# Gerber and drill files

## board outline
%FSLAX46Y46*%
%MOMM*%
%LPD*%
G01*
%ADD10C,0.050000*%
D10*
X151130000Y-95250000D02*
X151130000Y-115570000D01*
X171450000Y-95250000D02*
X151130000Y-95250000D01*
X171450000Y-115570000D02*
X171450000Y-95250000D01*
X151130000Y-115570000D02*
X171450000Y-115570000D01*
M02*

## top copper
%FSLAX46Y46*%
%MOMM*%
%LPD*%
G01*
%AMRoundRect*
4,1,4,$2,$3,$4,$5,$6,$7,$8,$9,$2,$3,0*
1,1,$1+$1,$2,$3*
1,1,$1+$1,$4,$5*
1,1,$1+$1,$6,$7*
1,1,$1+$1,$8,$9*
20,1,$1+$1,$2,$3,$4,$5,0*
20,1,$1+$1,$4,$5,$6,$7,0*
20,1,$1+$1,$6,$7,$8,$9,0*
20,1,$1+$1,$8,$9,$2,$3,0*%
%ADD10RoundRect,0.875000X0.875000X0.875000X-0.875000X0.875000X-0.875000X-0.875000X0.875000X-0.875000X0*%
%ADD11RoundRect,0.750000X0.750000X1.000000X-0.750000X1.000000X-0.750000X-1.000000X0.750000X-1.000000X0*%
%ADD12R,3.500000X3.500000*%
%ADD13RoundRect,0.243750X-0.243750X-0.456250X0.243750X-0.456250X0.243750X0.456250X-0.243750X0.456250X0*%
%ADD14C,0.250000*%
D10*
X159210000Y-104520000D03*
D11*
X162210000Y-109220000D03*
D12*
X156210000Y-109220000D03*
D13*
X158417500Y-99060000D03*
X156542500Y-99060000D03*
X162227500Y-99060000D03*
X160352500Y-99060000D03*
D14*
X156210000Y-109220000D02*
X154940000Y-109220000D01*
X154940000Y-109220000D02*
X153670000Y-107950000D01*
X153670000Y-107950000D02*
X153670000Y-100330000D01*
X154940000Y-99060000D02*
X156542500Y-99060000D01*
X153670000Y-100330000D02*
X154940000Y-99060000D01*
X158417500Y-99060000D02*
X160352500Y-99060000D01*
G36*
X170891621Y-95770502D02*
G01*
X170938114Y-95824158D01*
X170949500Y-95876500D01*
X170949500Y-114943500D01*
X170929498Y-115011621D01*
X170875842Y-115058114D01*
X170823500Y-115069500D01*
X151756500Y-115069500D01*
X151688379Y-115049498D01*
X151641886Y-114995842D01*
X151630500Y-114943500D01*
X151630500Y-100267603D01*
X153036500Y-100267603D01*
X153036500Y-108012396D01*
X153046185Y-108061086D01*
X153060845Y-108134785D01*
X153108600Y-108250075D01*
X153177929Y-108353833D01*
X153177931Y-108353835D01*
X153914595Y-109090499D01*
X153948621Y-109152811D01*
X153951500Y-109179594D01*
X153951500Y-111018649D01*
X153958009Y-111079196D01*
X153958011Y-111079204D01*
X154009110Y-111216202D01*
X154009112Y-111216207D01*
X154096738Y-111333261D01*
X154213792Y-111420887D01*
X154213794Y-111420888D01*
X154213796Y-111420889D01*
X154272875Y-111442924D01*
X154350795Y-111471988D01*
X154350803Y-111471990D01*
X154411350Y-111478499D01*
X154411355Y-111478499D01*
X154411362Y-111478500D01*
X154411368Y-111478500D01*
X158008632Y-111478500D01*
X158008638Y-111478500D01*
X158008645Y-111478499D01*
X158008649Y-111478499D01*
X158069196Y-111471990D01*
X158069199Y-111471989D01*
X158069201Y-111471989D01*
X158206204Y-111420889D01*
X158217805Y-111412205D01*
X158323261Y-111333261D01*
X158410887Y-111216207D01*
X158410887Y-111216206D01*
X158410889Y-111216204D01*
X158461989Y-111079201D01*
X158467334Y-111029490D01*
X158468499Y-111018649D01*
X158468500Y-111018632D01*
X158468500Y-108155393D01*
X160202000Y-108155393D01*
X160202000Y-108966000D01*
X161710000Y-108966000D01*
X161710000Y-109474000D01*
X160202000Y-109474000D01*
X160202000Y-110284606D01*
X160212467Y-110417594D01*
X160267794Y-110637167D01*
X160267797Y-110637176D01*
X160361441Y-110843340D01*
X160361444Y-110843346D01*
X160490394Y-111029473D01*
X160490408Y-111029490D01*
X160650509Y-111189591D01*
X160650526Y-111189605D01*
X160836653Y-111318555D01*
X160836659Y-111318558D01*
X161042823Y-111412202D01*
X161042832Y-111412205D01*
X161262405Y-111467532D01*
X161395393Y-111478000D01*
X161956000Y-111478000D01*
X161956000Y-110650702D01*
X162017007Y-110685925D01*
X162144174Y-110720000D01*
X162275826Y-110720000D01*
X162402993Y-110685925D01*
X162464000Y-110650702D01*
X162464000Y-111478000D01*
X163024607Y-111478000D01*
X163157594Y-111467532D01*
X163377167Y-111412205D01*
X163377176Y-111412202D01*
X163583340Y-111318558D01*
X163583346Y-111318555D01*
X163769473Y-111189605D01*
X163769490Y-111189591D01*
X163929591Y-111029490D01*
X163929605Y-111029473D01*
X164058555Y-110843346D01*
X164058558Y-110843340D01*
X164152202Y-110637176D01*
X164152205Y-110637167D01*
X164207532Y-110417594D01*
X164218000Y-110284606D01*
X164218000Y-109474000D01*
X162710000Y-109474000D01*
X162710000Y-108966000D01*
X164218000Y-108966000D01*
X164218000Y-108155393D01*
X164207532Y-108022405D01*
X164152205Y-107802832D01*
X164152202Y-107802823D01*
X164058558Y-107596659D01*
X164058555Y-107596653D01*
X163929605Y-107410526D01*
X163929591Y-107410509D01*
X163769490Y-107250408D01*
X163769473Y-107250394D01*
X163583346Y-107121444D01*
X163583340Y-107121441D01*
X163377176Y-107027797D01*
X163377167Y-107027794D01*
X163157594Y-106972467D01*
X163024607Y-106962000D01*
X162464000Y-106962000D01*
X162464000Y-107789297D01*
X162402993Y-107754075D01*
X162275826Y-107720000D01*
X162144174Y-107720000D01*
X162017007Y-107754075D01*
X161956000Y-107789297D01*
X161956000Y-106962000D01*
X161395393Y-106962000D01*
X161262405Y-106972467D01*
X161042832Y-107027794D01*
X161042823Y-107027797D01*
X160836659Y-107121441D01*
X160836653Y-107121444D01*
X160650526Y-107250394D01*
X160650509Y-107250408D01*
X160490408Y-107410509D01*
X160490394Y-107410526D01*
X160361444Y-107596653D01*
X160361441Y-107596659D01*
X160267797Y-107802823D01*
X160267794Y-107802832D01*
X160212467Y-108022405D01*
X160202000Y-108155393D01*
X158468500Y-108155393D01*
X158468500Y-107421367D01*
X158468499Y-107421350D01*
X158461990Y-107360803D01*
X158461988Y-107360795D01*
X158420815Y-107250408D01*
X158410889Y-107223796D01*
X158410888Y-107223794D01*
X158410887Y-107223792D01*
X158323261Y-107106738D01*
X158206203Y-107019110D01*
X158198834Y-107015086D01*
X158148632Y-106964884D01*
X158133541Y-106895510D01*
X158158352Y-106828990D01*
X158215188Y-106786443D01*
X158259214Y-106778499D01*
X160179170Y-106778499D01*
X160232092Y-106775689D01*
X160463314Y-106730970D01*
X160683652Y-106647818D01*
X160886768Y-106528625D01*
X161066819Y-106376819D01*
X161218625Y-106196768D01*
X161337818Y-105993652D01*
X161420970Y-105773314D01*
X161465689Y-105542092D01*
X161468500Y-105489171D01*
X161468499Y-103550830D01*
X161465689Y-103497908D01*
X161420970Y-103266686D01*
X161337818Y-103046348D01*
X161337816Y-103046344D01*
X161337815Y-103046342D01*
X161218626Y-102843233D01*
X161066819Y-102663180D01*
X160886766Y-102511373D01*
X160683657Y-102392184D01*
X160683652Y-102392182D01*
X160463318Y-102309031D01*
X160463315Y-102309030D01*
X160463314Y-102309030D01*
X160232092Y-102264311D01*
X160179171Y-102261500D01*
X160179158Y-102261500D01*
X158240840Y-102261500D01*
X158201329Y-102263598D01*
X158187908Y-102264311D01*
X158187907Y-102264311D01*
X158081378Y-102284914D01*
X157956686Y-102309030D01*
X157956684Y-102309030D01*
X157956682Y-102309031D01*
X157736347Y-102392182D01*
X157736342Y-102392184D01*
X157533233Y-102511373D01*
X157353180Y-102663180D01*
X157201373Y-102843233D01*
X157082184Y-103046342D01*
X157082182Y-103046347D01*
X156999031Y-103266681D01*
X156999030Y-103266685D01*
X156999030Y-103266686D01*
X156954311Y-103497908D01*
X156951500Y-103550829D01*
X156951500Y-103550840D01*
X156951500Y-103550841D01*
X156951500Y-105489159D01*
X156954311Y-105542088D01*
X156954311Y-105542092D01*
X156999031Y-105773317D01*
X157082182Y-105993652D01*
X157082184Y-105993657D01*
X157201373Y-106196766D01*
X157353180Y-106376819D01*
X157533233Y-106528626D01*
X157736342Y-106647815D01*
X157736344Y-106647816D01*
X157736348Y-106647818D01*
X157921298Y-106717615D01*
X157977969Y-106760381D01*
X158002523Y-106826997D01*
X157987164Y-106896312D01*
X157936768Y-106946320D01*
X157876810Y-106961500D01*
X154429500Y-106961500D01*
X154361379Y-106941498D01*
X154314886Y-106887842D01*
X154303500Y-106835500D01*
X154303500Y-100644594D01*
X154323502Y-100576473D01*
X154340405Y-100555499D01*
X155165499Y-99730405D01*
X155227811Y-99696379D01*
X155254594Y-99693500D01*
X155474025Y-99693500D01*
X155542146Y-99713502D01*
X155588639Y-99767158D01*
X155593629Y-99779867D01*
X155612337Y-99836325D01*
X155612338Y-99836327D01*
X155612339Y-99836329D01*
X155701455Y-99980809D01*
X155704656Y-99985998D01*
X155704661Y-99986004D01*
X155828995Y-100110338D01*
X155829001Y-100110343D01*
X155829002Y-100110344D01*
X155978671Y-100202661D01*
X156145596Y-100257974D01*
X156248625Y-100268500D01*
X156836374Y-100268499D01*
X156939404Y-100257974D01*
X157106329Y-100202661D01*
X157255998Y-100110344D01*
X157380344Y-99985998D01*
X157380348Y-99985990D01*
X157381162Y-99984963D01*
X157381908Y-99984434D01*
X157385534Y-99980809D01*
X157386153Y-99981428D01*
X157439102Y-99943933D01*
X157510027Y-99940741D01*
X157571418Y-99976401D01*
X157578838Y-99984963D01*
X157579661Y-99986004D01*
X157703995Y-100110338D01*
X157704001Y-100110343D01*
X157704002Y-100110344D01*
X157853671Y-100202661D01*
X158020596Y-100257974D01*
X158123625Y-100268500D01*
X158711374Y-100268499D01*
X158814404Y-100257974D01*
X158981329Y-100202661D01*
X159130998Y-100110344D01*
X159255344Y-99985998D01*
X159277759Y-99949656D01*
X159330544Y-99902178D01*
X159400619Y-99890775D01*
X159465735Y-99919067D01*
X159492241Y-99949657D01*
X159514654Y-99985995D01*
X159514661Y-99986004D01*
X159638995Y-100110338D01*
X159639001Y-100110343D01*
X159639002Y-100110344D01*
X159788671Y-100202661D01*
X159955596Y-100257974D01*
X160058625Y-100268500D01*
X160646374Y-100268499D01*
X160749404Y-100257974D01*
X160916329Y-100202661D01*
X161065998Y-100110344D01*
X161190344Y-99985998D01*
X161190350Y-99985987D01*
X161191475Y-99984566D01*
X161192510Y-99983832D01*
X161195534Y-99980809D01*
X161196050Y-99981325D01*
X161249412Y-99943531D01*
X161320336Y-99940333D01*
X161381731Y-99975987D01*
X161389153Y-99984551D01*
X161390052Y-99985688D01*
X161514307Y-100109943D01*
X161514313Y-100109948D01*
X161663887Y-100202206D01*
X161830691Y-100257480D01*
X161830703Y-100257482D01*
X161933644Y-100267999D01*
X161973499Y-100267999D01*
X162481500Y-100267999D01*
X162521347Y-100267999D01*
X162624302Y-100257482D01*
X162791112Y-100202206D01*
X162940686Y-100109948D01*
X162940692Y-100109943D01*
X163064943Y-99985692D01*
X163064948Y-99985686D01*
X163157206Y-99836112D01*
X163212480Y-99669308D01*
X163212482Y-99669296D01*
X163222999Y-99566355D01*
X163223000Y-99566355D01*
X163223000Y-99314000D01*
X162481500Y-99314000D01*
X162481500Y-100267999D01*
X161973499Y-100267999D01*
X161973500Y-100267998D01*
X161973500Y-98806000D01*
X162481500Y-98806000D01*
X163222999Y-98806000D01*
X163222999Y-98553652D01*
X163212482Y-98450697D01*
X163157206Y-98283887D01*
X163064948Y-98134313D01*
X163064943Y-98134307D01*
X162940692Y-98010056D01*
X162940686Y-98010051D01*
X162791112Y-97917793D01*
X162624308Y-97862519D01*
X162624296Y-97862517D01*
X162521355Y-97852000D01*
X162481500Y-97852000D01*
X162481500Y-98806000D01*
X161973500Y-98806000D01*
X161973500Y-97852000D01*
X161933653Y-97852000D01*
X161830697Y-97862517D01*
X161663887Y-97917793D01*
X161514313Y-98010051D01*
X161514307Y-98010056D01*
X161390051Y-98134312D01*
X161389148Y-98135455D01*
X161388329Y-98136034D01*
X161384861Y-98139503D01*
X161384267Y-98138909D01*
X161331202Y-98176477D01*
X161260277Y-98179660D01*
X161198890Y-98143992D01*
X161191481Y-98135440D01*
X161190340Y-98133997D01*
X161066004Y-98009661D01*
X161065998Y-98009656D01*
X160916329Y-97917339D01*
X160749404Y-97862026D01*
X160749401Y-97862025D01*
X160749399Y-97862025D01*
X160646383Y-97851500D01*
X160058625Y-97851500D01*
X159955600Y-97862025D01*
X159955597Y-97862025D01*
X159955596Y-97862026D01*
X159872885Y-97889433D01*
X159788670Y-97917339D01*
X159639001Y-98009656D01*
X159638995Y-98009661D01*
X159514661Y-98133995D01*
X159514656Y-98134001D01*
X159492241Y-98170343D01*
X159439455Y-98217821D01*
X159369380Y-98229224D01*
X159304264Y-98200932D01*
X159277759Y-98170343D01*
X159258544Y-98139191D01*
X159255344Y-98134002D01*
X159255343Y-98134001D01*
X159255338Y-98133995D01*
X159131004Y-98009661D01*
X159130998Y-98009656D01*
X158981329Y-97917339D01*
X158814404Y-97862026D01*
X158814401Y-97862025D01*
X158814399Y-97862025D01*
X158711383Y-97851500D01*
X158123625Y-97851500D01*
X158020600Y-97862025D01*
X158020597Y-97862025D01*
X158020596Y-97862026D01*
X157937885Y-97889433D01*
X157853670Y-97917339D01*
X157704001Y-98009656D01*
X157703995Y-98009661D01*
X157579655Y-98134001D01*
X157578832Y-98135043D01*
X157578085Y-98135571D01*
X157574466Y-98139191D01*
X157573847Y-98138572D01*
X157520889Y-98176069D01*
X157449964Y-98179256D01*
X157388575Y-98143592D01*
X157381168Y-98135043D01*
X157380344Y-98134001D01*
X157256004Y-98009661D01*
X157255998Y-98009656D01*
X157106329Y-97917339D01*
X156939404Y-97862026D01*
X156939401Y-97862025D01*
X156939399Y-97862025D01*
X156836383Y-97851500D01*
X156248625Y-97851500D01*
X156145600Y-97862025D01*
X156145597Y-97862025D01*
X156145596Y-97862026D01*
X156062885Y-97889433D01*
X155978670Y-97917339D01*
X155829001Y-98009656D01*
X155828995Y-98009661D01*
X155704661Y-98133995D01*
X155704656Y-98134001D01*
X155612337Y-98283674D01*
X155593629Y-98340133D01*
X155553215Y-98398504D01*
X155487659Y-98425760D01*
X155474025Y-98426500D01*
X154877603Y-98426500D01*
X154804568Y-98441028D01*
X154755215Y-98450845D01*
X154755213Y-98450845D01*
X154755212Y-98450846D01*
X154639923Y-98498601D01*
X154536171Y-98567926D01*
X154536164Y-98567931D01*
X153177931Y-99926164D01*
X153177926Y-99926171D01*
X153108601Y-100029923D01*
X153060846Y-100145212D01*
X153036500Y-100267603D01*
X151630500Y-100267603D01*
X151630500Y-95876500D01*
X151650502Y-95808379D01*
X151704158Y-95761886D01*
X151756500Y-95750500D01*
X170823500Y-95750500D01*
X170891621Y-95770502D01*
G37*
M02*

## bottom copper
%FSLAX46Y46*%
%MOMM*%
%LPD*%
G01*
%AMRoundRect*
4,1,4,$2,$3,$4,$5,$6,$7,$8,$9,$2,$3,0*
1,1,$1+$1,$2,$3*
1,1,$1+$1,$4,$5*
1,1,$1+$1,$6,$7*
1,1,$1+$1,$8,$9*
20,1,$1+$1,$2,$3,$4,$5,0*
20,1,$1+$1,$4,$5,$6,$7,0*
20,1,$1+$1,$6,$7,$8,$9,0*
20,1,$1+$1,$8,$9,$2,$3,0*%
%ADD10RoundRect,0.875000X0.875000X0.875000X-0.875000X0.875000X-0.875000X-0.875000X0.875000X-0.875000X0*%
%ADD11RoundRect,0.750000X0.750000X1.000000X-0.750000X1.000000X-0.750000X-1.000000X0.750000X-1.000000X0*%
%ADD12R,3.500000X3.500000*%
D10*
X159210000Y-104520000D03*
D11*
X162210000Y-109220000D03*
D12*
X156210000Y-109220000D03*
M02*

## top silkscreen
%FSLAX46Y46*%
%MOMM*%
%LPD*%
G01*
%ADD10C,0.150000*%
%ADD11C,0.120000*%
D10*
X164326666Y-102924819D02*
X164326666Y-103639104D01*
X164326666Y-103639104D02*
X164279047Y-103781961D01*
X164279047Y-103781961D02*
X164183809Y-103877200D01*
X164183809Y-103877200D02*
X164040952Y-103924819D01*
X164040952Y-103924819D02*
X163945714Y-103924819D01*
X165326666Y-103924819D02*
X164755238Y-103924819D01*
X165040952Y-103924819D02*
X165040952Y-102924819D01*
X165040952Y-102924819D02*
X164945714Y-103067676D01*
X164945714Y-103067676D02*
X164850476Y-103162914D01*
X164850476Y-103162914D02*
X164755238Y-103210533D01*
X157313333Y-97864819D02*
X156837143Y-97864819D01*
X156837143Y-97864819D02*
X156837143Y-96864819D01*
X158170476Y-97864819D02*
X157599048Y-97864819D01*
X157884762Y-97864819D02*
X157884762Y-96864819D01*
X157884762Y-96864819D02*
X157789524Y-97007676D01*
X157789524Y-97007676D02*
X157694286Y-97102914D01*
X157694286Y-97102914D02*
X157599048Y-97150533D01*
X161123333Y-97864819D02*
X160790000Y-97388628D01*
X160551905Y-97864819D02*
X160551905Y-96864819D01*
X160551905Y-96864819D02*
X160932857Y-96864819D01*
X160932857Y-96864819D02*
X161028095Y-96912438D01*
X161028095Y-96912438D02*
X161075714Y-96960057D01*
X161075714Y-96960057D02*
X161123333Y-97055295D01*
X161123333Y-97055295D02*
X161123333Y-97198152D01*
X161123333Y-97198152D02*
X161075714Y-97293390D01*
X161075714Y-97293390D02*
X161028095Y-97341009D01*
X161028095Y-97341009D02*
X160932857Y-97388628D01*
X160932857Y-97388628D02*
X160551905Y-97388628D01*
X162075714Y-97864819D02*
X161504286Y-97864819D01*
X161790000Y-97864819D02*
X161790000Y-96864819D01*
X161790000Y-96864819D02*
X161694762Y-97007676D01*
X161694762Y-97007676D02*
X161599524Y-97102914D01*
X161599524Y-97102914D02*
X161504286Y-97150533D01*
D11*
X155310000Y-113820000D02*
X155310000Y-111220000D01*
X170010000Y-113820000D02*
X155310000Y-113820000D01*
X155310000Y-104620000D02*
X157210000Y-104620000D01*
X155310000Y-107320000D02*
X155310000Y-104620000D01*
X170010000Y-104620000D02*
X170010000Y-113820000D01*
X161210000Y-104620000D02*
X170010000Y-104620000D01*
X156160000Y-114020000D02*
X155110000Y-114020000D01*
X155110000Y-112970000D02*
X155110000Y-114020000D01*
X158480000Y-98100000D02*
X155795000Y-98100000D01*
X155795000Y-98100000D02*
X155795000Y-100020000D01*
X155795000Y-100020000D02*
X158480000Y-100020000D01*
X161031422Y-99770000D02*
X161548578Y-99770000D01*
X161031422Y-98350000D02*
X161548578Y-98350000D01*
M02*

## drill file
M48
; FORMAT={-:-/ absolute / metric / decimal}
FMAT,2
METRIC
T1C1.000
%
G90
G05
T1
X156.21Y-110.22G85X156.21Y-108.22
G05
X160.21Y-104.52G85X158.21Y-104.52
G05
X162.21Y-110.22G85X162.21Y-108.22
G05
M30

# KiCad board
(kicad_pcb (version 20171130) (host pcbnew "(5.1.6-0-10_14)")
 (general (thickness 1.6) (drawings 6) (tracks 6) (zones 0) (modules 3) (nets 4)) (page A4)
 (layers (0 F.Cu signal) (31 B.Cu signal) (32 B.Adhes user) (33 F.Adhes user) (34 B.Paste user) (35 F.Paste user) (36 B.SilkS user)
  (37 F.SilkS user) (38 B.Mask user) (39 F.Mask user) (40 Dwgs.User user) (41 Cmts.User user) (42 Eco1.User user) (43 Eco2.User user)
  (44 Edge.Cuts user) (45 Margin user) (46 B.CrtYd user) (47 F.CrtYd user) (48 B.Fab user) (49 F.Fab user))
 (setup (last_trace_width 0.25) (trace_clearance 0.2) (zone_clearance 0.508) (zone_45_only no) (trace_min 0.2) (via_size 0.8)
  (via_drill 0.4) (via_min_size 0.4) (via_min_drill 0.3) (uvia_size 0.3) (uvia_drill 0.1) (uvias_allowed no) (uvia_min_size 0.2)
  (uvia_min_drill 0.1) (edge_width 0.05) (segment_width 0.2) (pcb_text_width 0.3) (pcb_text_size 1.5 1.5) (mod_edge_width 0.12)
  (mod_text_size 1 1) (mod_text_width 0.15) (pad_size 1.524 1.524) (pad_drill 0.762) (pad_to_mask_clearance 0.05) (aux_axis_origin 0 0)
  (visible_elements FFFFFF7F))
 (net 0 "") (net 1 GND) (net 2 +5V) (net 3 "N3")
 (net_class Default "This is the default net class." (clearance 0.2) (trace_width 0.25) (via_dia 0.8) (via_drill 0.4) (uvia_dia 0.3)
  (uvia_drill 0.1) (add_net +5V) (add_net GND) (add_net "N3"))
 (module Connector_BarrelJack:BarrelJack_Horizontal (layer F.Cu) (at 156.21 109.22 180)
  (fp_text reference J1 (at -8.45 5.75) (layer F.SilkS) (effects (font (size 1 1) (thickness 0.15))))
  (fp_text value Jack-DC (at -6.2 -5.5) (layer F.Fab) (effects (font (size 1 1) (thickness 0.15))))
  (fp_line (start 0.9 -4.6) (end 0.9 -2) (layer F.SilkS) (width 0.12))
  (fp_line (start -13.8 -4.6) (end 0.9 -4.6) (layer F.SilkS) (width 0.12))
  (fp_line (start 0.9 4.6) (end -1 4.6) (layer F.SilkS) (width 0.12))
  (fp_line (start 0.9 1.9) (end 0.9 4.6) (layer F.SilkS) (width 0.12))
  (fp_line (start -13.8 4.6) (end -13.8 -4.6) (layer F.SilkS) (width 0.12))
  (fp_line (start -5 4.6) (end -13.8 4.6) (layer F.SilkS) (width 0.12))
  (fp_line (start 0.05 -4.8) (end 1.1 -4.8) (layer F.SilkS) (width 0.12))
  (fp_line (start 1.1 -3.75) (end 1.1 -4.8) (layer F.SilkS) (width 0.12))
  (pad 3 thru_hole roundrect (at -3 4.7 180) (size 3.5 3.5) (drill oval 3 1) (layers *.Cu *.Mask) (roundrect_rratio 0.25))
  (pad 2 thru_hole roundrect (at -6 0 180) (size 3 3.5) (drill oval 1 3) (layers *.Cu *.Mask) (roundrect_rratio 0.25) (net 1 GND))
  (pad 1 thru_hole rect (at 0 0 180) (size 3.5 3.5) (drill oval 1 3) (layers *.Cu *.Mask) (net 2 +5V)))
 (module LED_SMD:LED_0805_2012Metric (layer F.Cu) (at 157.48 99.06)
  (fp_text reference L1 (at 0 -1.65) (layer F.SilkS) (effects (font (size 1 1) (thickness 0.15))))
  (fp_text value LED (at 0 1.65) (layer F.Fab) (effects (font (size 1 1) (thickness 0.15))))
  (fp_line (start 1 -0.96) (end -1.685 -0.96) (layer F.SilkS) (width 0.12))
  (fp_line (start -1.685 -0.96) (end -1.685 0.96) (layer F.SilkS) (width 0.12))
  (fp_line (start -1.685 0.96) (end 1 0.96) (layer F.SilkS) (width 0.12))
  (pad 2 smd roundrect (at 0.9375 0) (size 0.975 1.4) (layers F.Cu F.Paste F.Mask) (roundrect_rratio 0.25) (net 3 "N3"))
  (pad 1 smd roundrect (at -0.9375 0) (size 0.975 1.4) (layers F.Cu F.Paste F.Mask) (roundrect_rratio 0.25) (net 2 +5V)))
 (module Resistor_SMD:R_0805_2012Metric (layer F.Cu) (at 161.29 99.06)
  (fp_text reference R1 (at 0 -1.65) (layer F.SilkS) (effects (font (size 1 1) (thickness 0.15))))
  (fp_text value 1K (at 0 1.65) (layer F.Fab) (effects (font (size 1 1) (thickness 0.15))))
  (fp_line (start -0.258578 0.71) (end 0.258578 0.71) (layer F.SilkS) (width 0.12))
  (fp_line (start -0.258578 -0.71) (end 0.258578 -0.71) (layer F.SilkS) (width 0.12))
  (pad 2 smd roundrect (at 0.9375 0) (size 0.975 1.4) (layers F.Cu F.Paste F.Mask) (roundrect_rratio 0.25) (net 1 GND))
  (pad 1 smd roundrect (at -0.9375 0) (size 0.975 1.4) (layers F.Cu F.Paste F.Mask) (roundrect_rratio 0.25) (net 3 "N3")))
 (gr_line (start 151.13 95.25) (end 151.13 115.57) (layer Edge.Cuts) (width 0.05))
 (gr_line (start 171.45 95.25) (end 151.13 95.25) (layer Edge.Cuts) (width 0.05))
 (gr_line (start 171.45 115.57) (end 171.45 95.25) (layer Edge.Cuts) (width 0.05))
 (gr_line (start 151.13 115.57) (end 171.45 115.57) (layer Edge.Cuts) (width 0.05))
 (segment (start 156.21 109.22) (end 154.94 109.22) (width 0.25) (layer F.Cu) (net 2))
 (segment (start 154.94 109.22) (end 153.67 107.95) (width 0.25) (layer F.Cu) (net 2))
 (segment (start 153.67 107.95) (end 153.67 100.33) (width 0.25) (layer F.Cu) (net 2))
 (segment (start 154.94 99.06) (end 156.5425 99.06) (width 0.25) (layer F.Cu) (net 2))
 (segment (start 153.67 100.33) (end 154.94 99.06) (width 0.25) (layer F.Cu) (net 2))
 (segment (start 158.4175 99.06) (end 160.3525 99.06) (width 0.25) (layer F.Cu) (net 3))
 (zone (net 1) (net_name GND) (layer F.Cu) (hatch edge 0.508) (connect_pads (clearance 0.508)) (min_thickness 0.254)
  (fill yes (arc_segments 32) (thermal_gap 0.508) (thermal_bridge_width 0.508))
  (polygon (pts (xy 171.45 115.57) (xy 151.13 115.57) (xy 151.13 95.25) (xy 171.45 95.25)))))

